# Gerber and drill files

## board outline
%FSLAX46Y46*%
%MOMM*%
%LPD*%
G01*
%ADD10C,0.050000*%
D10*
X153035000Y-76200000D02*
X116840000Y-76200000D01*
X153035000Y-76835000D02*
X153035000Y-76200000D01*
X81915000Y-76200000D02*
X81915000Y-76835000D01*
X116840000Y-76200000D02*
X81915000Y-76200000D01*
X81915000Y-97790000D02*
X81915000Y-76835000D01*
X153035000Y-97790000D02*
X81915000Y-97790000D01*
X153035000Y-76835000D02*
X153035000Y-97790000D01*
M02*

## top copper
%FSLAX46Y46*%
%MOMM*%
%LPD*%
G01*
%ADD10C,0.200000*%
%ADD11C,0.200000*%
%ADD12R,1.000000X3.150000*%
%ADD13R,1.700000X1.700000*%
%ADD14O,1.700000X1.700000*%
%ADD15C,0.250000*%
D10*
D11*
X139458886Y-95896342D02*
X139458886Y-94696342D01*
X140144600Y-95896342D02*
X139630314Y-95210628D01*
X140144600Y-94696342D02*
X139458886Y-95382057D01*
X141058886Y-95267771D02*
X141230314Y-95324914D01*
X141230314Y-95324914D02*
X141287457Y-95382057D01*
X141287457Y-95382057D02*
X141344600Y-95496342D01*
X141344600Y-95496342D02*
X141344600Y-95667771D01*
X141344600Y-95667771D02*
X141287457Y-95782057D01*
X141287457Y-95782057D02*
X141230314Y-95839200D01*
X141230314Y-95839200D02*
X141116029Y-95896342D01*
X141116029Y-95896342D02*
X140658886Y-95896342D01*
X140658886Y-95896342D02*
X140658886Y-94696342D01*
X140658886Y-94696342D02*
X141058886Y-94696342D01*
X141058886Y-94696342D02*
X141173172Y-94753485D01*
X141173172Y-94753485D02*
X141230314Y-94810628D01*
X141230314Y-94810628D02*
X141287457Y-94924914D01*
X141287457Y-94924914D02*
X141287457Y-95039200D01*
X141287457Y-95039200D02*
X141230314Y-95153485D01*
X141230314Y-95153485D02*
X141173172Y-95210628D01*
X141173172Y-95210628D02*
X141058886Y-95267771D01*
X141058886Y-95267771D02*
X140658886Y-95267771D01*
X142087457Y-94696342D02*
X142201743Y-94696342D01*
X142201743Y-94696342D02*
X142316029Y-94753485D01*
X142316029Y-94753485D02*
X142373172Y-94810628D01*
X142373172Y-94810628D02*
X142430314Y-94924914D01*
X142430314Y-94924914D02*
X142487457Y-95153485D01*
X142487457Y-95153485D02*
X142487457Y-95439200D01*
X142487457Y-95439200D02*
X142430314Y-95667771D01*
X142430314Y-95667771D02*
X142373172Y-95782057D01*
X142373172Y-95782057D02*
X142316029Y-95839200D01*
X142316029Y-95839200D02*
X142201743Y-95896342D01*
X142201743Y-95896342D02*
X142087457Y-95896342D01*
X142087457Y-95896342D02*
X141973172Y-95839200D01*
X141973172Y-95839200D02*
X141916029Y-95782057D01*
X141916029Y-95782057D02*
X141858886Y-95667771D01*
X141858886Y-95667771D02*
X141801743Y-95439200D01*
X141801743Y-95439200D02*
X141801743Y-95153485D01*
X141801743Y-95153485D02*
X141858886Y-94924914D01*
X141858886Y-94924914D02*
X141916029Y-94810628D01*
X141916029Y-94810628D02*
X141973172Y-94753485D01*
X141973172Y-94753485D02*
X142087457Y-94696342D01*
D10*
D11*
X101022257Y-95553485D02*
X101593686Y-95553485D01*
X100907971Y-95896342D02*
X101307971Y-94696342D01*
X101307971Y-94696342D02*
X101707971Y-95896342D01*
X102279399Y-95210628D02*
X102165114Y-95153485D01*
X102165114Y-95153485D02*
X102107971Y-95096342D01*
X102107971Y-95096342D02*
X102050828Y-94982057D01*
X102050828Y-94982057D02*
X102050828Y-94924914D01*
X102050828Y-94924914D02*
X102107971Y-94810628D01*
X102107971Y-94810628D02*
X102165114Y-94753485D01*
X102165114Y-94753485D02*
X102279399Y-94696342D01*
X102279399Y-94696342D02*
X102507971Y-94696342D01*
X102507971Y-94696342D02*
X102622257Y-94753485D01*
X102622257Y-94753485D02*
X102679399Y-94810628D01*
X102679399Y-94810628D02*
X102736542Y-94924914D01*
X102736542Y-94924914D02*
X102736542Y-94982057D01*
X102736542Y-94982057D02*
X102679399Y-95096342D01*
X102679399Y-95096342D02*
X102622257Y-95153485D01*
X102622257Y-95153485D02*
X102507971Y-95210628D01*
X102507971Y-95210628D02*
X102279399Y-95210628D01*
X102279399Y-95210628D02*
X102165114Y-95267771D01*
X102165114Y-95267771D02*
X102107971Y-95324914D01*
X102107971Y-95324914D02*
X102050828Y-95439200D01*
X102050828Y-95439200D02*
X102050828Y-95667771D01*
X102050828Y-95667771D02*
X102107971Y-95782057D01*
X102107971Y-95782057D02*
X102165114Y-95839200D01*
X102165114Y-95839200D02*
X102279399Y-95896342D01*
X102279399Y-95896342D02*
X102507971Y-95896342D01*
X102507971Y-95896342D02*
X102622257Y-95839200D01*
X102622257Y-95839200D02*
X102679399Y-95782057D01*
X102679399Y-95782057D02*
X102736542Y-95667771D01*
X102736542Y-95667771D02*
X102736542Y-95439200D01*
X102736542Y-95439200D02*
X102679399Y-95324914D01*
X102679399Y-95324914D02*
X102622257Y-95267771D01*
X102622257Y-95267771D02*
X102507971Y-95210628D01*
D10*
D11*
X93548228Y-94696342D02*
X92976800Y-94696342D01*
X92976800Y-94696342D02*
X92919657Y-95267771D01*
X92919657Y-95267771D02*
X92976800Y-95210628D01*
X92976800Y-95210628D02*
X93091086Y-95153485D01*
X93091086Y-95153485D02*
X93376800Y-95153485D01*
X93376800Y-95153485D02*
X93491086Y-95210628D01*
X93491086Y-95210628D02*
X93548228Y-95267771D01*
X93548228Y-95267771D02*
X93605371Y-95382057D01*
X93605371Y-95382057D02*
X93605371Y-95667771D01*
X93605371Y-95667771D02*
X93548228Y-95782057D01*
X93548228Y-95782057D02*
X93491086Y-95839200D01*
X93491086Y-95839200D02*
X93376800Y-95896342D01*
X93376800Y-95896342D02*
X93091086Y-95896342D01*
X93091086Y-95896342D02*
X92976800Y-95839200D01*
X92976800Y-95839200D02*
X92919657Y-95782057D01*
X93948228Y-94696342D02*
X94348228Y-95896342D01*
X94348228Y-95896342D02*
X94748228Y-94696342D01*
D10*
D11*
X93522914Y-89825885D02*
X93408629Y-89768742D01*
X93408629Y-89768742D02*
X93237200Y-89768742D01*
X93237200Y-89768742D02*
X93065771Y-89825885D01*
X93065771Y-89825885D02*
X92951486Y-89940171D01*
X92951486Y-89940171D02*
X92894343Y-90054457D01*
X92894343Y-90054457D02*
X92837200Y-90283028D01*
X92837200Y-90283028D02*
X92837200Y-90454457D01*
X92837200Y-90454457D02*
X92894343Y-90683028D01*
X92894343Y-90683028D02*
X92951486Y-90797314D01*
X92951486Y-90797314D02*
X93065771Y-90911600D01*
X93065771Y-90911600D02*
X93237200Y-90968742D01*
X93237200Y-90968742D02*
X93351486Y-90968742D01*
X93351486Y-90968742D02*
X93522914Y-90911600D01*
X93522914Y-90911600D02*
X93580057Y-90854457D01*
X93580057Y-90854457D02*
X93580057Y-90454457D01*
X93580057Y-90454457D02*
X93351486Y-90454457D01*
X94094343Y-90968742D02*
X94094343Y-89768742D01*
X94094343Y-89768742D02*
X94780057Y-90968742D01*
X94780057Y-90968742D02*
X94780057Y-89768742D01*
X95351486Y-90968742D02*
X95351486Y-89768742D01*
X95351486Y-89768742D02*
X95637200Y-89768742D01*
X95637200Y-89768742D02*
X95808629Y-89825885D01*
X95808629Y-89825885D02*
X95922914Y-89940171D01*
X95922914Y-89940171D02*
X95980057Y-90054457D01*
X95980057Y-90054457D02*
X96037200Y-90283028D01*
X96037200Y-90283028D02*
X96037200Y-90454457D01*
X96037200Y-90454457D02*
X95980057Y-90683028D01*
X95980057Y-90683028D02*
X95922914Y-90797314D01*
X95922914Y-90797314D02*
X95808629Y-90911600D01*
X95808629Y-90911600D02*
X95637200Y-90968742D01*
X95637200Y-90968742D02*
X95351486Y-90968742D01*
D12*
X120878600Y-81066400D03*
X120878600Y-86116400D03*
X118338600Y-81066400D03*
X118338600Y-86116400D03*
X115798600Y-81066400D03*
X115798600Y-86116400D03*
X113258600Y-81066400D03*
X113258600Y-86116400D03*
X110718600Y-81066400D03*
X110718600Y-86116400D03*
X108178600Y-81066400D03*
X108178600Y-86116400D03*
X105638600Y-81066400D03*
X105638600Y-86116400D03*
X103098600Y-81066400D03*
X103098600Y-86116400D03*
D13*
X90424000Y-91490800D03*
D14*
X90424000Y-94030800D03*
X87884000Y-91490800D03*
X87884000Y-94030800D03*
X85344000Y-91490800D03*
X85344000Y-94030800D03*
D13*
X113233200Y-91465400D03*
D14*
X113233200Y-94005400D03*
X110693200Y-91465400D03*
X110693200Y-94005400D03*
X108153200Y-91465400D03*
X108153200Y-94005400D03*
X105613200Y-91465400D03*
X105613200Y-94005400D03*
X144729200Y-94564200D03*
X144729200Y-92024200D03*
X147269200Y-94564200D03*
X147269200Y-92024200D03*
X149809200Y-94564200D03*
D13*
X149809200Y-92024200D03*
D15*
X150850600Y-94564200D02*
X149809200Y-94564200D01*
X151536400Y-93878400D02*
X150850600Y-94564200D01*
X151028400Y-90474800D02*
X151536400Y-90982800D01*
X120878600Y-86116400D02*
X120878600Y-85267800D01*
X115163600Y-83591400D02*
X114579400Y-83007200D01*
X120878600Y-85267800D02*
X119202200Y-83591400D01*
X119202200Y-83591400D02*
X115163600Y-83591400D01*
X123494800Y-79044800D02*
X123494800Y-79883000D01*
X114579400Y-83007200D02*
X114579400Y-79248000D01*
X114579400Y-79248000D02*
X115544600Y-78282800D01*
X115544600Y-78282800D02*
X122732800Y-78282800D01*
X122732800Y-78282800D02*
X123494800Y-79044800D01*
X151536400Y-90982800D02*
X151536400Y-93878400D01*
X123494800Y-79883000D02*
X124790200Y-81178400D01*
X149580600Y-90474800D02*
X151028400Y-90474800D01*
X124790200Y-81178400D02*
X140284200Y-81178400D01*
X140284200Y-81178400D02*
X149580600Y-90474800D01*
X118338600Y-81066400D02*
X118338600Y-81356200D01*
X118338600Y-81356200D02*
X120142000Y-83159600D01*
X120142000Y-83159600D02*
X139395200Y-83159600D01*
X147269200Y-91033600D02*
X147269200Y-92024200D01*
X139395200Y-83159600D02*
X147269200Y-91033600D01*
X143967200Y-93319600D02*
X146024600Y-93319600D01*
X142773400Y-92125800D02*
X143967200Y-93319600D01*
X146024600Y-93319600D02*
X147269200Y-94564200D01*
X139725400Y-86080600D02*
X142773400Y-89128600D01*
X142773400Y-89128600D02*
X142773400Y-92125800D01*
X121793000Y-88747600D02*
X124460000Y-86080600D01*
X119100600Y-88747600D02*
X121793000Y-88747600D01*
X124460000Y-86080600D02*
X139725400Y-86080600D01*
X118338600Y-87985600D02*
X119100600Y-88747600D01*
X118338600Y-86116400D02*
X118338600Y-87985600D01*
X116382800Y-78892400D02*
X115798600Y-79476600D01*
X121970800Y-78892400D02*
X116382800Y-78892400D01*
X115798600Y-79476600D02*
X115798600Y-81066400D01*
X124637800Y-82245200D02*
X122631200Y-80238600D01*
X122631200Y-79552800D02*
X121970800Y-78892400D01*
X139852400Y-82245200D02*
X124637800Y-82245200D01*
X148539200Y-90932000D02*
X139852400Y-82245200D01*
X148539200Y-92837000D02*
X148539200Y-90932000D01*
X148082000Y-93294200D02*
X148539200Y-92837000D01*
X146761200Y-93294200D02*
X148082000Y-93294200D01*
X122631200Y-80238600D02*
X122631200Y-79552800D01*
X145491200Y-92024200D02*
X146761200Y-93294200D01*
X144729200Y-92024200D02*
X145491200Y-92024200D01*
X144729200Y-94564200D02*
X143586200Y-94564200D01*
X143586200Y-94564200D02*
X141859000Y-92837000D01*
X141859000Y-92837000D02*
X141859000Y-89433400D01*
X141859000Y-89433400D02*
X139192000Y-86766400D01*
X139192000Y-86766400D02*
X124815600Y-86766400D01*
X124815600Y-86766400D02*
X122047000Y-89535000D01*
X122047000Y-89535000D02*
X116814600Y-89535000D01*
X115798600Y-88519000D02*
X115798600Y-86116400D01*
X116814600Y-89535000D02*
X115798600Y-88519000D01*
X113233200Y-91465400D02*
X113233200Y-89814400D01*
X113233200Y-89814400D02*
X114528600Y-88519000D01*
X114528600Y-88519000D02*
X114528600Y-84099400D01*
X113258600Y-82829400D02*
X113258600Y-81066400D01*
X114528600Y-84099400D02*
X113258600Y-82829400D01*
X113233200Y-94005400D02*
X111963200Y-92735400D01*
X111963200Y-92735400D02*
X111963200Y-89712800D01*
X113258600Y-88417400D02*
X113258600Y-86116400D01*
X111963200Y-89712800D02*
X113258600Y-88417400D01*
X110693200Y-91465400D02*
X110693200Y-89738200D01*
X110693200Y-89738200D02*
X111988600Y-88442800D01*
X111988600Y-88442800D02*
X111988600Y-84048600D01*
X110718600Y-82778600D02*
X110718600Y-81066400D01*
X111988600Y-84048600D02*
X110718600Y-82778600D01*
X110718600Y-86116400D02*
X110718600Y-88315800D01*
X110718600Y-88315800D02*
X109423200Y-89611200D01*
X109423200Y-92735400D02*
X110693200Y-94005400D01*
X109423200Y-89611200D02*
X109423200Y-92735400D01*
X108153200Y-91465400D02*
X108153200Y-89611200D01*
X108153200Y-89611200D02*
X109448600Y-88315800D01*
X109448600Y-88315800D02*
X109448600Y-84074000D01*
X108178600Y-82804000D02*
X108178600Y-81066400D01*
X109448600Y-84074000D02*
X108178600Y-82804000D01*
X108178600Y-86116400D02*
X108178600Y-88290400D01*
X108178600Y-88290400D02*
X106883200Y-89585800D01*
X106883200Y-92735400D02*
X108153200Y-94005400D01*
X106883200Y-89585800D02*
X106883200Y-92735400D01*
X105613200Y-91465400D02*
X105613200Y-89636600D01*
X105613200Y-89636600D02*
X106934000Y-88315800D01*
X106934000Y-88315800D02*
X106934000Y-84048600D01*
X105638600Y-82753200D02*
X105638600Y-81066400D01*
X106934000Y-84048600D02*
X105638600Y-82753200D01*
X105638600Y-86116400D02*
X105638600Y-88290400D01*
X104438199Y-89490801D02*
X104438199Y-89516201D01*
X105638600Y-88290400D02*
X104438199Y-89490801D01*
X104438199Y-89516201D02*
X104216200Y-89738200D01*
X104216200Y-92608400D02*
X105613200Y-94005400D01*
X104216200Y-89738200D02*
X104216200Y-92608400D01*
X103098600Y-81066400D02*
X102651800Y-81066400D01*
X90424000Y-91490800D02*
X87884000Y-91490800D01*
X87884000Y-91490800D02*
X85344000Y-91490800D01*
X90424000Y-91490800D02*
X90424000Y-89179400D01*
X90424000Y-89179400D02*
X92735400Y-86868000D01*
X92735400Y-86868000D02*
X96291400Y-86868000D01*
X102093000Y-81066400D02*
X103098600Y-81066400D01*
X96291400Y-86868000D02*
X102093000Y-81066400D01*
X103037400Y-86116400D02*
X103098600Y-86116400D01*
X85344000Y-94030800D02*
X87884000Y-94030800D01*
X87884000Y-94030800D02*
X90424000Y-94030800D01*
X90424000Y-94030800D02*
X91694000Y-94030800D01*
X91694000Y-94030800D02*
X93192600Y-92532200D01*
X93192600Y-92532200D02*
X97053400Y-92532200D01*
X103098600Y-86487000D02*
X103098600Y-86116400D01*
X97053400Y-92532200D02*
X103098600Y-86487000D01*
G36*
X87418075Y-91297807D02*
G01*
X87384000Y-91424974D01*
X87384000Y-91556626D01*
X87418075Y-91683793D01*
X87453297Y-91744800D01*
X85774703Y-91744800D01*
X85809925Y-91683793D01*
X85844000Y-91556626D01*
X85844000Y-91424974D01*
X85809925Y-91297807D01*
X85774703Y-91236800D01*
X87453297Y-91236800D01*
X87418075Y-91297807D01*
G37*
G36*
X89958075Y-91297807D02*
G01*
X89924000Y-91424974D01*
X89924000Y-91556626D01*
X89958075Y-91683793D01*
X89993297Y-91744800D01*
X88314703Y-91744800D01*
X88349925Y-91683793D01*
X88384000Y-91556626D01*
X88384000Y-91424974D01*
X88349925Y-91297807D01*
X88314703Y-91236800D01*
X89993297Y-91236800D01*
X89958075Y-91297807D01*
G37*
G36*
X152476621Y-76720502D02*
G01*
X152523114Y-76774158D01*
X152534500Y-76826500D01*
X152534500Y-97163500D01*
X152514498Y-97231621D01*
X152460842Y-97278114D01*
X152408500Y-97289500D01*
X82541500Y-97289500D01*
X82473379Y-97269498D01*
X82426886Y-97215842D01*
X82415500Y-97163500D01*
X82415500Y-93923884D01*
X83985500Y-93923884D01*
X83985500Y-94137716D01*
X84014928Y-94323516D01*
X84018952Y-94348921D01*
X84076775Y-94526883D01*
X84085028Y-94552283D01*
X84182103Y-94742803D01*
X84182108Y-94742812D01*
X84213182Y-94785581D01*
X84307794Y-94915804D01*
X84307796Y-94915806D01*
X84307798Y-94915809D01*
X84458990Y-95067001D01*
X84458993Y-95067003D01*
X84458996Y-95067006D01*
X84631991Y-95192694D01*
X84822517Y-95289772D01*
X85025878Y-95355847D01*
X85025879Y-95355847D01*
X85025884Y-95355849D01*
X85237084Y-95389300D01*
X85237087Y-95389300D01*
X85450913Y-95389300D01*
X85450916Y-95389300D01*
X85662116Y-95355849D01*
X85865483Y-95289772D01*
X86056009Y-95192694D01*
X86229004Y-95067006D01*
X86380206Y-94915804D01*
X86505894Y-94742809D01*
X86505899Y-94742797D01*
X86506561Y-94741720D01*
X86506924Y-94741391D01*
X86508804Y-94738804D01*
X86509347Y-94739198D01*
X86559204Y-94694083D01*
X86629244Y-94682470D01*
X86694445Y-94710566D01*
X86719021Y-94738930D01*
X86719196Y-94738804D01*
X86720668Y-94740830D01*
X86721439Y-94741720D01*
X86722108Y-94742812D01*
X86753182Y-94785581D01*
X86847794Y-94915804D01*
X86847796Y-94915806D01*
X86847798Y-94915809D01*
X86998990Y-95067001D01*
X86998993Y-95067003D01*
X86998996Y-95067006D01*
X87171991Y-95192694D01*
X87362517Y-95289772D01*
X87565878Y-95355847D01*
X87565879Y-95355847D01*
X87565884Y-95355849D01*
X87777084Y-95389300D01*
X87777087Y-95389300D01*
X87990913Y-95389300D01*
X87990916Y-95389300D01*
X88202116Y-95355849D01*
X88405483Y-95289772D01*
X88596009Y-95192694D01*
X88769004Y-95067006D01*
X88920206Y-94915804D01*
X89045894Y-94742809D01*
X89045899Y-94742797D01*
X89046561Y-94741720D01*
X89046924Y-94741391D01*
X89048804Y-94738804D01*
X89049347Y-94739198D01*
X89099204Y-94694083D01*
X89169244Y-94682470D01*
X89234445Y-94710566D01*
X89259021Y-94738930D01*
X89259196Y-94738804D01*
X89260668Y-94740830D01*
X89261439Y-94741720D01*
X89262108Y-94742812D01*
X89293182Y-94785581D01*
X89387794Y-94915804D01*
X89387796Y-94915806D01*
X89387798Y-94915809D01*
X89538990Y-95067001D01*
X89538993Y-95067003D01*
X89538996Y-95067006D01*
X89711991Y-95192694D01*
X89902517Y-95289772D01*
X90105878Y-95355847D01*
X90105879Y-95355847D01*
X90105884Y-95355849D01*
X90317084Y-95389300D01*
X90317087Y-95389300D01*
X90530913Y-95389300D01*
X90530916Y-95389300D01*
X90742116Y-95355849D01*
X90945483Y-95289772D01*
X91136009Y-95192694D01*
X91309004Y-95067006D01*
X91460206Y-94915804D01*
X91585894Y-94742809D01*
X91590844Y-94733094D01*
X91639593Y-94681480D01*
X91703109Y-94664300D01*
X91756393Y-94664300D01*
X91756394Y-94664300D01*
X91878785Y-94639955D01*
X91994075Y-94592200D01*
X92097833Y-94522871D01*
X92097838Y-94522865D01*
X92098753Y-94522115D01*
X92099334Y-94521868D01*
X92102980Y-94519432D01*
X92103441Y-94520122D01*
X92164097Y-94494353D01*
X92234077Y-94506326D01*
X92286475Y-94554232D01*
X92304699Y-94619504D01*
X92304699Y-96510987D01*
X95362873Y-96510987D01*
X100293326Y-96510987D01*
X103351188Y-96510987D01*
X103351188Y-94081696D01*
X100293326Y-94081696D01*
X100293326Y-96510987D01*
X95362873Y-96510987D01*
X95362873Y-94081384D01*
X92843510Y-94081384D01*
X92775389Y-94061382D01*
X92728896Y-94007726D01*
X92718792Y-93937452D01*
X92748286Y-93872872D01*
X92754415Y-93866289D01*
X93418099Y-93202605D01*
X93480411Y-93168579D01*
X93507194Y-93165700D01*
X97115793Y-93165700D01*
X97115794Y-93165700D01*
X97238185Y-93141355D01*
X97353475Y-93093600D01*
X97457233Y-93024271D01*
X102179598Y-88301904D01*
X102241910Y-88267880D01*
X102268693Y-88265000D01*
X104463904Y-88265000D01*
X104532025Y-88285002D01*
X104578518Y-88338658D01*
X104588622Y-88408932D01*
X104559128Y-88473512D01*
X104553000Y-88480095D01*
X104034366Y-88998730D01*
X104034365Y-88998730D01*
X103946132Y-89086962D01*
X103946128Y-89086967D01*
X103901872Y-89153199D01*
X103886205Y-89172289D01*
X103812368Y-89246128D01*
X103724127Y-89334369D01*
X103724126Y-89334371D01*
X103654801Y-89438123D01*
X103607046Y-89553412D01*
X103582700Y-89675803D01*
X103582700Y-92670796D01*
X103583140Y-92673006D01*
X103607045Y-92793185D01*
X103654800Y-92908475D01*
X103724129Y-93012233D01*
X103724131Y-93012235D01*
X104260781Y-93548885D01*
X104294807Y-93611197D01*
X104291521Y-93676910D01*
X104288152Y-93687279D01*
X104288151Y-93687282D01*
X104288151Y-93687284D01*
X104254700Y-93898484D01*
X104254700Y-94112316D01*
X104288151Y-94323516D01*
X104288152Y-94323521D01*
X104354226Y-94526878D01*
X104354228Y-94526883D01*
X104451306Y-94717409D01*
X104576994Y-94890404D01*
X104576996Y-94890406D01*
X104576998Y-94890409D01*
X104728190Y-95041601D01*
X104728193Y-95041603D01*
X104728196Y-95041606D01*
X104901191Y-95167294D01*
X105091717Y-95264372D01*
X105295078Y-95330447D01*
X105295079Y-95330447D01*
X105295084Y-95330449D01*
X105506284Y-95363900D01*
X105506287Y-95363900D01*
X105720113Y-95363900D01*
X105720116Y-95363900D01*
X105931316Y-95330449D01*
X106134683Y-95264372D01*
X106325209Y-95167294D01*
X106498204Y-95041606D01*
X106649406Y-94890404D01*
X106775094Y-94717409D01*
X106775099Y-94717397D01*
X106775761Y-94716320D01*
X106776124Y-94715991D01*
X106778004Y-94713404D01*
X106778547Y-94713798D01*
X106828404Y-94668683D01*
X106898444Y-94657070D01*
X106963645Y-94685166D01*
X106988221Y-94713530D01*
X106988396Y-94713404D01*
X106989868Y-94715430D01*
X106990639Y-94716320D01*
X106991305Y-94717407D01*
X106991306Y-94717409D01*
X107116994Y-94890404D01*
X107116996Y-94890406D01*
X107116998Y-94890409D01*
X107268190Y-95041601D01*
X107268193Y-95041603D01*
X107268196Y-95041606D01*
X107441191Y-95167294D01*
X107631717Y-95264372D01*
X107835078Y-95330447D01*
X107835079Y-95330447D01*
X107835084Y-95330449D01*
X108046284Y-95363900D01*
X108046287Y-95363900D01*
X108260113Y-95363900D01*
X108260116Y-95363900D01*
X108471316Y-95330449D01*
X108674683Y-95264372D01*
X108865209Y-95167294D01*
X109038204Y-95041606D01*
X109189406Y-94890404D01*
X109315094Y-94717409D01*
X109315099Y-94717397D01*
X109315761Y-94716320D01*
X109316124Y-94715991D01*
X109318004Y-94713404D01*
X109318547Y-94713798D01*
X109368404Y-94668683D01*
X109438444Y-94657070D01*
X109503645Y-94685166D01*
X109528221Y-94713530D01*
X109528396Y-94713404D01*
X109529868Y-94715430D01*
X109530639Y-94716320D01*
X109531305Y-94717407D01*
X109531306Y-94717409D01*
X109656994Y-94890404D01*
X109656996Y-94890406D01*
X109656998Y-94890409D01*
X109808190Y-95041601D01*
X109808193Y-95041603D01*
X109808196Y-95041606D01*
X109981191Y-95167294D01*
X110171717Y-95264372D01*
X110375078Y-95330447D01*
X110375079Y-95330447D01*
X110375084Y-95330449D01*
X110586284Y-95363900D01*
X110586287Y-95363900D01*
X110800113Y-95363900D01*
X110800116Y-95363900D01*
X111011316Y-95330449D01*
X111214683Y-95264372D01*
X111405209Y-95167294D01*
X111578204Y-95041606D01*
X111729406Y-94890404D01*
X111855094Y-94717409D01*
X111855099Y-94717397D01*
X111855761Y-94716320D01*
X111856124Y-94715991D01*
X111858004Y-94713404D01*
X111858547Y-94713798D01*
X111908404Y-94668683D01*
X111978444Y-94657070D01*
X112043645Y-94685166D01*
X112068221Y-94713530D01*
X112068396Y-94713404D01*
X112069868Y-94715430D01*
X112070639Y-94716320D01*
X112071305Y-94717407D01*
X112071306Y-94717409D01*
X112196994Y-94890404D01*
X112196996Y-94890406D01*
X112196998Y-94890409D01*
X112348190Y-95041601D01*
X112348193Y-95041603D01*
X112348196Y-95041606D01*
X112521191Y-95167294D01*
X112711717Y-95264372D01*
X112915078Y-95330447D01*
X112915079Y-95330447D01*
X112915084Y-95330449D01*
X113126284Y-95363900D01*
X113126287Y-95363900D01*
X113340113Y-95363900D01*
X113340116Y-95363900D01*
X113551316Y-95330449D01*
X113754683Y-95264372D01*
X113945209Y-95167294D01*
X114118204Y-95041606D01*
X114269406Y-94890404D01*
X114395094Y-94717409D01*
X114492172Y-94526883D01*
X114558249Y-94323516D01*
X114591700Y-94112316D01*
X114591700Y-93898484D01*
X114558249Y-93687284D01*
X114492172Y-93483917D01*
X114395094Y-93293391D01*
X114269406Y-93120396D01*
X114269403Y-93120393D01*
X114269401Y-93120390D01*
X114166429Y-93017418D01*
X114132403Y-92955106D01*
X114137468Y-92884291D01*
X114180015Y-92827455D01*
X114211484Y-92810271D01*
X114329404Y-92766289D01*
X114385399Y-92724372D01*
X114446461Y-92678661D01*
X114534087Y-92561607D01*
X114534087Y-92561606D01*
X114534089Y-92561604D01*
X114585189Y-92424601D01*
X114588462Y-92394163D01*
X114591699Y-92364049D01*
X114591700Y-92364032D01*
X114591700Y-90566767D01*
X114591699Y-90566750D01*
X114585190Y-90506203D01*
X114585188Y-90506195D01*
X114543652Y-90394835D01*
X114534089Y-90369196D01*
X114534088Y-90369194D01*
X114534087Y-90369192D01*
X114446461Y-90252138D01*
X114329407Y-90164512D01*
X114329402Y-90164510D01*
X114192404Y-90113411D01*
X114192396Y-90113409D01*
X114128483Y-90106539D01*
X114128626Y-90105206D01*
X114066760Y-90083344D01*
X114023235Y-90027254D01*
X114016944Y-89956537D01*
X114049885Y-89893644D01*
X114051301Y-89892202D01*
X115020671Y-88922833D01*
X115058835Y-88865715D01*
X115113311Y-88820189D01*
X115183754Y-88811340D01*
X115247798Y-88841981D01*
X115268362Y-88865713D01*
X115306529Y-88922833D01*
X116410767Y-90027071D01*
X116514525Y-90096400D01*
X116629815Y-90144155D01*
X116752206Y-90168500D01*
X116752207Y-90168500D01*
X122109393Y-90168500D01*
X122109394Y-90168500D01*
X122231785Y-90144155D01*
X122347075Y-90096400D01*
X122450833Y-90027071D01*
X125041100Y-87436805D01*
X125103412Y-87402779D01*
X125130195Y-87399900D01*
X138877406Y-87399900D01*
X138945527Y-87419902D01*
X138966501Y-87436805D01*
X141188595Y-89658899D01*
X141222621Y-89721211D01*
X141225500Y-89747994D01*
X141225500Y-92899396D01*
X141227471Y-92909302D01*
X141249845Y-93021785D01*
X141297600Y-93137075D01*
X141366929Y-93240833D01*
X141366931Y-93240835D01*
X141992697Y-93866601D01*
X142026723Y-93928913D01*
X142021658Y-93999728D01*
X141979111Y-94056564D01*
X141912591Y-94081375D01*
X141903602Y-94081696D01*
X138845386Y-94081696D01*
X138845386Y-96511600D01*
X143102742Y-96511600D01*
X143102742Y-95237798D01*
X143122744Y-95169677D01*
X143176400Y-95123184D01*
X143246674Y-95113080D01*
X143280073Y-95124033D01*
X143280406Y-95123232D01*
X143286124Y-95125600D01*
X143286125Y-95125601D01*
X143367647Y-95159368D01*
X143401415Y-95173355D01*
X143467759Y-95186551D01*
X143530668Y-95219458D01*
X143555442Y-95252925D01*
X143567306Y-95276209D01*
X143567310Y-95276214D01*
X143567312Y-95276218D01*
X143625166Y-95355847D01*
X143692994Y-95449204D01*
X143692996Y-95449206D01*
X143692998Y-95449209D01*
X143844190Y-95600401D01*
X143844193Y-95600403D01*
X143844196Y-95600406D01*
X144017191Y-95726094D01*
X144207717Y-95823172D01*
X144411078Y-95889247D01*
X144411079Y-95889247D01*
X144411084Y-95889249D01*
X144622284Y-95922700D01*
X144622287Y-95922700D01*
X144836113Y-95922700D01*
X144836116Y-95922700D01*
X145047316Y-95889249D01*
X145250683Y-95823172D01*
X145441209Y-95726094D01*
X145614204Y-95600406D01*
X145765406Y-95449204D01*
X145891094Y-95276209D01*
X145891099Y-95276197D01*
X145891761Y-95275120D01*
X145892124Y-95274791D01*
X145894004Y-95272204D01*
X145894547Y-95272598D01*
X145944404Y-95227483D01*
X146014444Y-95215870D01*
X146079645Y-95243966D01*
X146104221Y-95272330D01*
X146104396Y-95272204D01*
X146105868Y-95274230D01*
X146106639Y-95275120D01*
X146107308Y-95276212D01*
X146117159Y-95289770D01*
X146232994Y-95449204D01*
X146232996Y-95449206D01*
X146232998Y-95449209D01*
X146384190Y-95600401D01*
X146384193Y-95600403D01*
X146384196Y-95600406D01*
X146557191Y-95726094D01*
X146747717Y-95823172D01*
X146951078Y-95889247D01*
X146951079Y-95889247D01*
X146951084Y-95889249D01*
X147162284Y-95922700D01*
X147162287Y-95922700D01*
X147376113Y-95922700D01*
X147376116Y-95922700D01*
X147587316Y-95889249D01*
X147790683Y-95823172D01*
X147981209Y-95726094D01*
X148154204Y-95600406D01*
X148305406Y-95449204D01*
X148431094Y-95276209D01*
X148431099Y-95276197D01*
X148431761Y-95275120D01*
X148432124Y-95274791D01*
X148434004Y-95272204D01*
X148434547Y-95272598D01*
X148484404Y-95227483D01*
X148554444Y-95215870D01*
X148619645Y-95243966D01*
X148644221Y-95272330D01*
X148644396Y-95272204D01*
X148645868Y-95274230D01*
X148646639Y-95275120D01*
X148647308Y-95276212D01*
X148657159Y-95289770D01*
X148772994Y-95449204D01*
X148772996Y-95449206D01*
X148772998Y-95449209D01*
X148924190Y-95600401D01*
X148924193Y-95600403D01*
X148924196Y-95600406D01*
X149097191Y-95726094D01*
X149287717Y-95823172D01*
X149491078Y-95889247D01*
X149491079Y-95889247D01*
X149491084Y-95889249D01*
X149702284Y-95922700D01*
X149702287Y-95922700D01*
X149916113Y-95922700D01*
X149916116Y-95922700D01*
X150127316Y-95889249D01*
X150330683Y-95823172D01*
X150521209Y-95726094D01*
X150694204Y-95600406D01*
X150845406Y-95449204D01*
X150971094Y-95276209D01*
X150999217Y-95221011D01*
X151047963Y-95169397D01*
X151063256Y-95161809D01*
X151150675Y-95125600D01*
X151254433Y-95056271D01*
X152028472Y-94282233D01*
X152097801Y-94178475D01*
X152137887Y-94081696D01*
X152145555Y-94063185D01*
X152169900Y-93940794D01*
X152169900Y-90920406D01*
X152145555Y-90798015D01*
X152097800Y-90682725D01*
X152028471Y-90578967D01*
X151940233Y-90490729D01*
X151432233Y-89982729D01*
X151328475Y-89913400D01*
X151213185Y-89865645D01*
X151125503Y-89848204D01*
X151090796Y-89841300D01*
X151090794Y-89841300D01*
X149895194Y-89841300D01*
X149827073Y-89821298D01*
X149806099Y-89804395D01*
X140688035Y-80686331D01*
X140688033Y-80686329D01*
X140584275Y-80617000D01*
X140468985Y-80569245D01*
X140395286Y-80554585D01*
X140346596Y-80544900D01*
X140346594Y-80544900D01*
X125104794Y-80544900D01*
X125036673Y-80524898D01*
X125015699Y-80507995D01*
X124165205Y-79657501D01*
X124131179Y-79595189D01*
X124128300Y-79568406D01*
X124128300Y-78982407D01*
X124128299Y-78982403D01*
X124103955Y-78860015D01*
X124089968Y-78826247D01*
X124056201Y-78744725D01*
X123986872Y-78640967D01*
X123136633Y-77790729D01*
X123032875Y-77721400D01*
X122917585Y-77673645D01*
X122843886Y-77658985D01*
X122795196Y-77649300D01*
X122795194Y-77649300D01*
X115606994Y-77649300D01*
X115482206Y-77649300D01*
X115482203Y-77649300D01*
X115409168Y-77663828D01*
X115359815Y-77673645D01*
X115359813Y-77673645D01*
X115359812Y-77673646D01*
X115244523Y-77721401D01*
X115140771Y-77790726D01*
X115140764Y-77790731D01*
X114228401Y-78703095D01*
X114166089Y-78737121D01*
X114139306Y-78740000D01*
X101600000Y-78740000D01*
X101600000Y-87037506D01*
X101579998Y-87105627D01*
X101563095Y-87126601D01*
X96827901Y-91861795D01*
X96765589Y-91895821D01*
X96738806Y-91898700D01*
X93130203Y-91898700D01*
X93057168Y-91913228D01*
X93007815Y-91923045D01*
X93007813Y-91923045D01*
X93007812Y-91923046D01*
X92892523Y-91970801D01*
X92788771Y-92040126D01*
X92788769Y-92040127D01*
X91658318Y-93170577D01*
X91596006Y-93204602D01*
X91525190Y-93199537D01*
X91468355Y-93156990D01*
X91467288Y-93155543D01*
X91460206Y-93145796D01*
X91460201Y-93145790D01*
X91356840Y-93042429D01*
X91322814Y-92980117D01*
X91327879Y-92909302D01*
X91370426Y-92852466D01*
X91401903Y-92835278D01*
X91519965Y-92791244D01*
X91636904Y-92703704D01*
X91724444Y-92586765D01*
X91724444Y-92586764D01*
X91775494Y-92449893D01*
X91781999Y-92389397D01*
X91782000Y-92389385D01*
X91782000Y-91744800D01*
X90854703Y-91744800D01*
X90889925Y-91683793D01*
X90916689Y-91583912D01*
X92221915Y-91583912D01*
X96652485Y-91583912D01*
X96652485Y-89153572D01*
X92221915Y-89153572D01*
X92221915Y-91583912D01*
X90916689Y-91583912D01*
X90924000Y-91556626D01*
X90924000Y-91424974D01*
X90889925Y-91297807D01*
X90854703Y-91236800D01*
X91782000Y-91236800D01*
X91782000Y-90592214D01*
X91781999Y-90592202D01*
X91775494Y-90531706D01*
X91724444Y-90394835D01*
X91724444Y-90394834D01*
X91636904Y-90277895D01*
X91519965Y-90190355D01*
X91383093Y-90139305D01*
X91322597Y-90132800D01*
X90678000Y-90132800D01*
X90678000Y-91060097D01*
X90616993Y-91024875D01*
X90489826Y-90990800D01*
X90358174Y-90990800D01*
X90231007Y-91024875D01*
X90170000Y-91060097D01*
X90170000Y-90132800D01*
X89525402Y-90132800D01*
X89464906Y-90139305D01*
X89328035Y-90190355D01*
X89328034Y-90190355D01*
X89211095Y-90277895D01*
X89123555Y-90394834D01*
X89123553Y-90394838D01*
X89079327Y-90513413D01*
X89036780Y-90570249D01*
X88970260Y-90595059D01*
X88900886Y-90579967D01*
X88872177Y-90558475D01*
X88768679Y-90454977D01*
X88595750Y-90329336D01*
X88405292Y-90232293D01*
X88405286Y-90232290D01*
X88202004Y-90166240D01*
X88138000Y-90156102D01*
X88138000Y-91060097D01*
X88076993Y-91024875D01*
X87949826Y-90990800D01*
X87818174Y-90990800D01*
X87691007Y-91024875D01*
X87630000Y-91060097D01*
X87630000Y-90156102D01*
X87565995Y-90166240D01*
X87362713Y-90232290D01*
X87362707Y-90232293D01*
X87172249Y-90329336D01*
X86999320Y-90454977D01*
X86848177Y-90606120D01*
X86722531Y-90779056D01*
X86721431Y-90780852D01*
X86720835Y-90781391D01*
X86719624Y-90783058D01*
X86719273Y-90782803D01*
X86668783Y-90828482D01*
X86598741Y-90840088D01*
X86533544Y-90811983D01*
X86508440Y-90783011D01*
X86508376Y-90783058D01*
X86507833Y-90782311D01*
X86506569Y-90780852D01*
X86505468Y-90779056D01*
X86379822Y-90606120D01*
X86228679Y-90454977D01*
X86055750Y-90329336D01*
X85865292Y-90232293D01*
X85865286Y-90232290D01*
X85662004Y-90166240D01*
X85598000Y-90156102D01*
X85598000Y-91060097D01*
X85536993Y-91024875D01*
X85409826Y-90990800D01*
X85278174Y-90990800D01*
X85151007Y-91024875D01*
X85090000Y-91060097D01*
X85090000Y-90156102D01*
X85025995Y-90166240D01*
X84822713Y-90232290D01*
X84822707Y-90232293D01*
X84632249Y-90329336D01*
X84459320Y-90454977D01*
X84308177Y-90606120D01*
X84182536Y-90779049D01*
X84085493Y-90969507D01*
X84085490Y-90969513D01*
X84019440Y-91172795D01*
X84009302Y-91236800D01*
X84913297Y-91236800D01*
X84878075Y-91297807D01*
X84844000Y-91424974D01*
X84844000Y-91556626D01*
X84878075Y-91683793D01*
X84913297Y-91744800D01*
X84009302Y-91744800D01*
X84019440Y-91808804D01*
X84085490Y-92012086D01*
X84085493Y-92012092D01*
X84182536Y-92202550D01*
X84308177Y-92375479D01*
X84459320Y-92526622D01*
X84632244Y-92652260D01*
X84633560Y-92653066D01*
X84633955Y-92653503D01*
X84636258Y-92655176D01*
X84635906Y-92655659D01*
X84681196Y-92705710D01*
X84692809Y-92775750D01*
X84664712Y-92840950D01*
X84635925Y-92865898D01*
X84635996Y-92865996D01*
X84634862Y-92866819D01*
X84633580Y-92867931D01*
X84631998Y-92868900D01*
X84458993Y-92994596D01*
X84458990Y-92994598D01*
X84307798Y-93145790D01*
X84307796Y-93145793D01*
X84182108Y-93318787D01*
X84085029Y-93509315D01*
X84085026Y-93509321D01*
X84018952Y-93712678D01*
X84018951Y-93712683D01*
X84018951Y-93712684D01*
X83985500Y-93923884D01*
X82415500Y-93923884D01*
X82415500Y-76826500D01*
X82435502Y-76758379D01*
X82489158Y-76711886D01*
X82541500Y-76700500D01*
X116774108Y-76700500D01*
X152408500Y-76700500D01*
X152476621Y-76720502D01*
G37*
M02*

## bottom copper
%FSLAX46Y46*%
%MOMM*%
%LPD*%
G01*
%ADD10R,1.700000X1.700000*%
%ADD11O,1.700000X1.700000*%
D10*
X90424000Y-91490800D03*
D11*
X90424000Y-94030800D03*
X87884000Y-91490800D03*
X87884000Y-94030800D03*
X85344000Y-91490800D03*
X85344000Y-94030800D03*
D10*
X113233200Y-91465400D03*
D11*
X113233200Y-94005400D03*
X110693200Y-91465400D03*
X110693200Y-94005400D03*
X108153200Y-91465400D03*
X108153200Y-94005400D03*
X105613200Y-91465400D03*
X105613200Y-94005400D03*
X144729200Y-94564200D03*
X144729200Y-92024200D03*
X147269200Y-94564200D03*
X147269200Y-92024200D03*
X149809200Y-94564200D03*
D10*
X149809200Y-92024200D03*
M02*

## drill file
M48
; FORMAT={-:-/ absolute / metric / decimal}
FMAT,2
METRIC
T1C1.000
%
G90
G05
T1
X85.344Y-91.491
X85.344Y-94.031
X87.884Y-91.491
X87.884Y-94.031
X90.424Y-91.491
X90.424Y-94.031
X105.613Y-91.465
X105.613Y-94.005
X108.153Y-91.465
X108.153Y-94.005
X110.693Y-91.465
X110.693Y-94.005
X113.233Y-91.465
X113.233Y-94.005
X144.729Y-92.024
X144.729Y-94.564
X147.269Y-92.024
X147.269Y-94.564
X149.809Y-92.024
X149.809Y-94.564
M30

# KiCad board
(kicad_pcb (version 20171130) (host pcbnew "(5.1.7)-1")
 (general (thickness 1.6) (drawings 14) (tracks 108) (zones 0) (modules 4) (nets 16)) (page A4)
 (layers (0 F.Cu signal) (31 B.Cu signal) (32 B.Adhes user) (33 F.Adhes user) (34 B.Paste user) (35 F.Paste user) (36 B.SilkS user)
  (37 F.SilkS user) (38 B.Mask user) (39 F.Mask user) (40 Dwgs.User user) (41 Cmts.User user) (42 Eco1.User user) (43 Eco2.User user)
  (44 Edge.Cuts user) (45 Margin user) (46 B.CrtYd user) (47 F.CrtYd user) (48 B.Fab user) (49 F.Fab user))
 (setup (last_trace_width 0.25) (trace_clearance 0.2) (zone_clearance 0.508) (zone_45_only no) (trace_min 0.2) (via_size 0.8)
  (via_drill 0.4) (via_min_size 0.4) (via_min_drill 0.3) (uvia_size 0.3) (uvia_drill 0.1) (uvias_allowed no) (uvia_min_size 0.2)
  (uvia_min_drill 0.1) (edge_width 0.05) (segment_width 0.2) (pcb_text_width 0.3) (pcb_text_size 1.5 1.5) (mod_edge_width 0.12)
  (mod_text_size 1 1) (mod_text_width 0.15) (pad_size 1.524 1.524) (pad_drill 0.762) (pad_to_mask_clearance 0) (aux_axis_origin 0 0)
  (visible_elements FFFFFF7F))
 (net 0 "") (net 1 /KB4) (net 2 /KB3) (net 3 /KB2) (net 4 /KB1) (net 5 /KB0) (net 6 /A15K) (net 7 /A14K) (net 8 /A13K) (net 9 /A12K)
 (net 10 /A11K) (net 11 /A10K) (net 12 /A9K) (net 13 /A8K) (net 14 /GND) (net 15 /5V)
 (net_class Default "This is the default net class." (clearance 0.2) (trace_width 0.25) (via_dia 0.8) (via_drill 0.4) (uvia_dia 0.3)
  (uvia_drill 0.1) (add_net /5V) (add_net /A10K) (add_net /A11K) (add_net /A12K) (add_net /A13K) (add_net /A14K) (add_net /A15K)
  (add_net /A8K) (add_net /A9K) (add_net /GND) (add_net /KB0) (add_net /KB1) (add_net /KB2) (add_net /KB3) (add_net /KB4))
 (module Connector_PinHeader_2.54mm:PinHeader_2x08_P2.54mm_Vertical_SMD (layer F.Cu) (at 111.9886 83.5914 270)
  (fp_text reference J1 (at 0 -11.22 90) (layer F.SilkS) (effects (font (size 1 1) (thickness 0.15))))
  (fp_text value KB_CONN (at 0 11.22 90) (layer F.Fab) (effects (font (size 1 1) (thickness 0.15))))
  (pad 1 smd rect (at -2.525 -8.89 270) (size 3.15 1) (layers F.Cu F.Paste F.Mask))
  (pad 2 smd rect (at 2.525 -8.89 270) (size 3.15 1) (layers F.Cu F.Paste F.Mask) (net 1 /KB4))
  (pad 3 smd rect (at -2.525 -6.35 270) (size 3.15 1) (layers F.Cu F.Paste F.Mask) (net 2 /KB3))
  (pad 4 smd rect (at 2.525 -6.35 270) (size 3.15 1) (layers F.Cu F.Paste F.Mask) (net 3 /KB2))
  (pad 5 smd rect (at -2.525 -3.81 270) (size 3.15 1) (layers F.Cu F.Paste F.Mask) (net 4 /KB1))
  (pad 6 smd rect (at 2.525 -3.81 270) (size 3.15 1) (layers F.Cu F.Paste F.Mask) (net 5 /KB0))
  (pad 7 smd rect (at -2.525 -1.27 270) (size 3.15 1) (layers F.Cu F.Paste F.Mask) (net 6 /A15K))
  (pad 8 smd rect (at 2.525 -1.27 270) (size 3.15 1) (layers F.Cu F.Paste F.Mask) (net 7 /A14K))
  (pad 9 smd rect (at -2.525 1.27 270) (size 3.15 1) (layers F.Cu F.Paste F.Mask) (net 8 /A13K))
  (pad 10 smd rect (at 2.525 1.27 270) (size 3.15 1) (layers F.Cu F.Paste F.Mask) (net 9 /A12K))
  (pad 11 smd rect (at -2.525 3.81 270) (size 3.15 1) (layers F.Cu F.Paste F.Mask) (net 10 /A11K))
  (pad 12 smd rect (at 2.525 3.81 270) (size 3.15 1) (layers F.Cu F.Paste F.Mask) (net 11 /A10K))
  (pad 13 smd rect (at -2.525 6.35 270) (size 3.15 1) (layers F.Cu F.Paste F.Mask) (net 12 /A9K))
  (pad 14 smd rect (at 2.525 6.35 270) (size 3.15 1) (layers F.Cu F.Paste F.Mask) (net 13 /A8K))
  (pad 15 smd rect (at -2.525 8.89 270) (size 3.15 1) (layers F.Cu F.Paste F.Mask) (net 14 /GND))
  (pad 16 smd rect (at 2.525 8.89 270) (size 3.15 1) (layers F.Cu F.Paste F.Mask) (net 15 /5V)))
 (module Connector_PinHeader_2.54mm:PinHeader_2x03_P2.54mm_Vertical (layer F.Cu) (at 90.424 91.4908 270)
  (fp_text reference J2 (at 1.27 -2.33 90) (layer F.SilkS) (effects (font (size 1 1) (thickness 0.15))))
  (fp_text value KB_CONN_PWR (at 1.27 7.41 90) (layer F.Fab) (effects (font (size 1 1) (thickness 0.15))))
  (pad 1 thru_hole rect (at 0 0 270) (size 1.7 1.7) (drill 1) (layers *.Cu *.Mask) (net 14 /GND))
  (pad 2 thru_hole oval (at 2.54 0 270) (size 1.7 1.7) (drill 1) (layers *.Cu *.Mask) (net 15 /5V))
  (pad 3 thru_hole oval (at 0 2.54 270) (size 1.7 1.7) (drill 1) (layers *.Cu *.Mask) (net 14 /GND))
  (pad 4 thru_hole oval (at 2.54 2.54 270) (size 1.7 1.7) (drill 1) (layers *.Cu *.Mask) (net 15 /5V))
  (pad 5 thru_hole oval (at 0 5.08 270) (size 1.7 1.7) (drill 1) (layers *.Cu *.Mask) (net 14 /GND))
  (pad 6 thru_hole oval (at 2.54 5.08 270) (size 1.7 1.7) (drill 1) (layers *.Cu *.Mask) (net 15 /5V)))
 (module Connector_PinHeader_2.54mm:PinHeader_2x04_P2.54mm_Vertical (layer F.Cu) (at 113.2332 91.4654 270)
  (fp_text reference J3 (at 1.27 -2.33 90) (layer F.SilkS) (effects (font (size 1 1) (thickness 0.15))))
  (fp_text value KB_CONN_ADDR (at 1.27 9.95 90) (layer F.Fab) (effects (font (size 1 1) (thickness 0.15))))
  (pad 1 thru_hole rect (at 0 0 270) (size 1.7 1.7) (drill 1) (layers *.Cu *.Mask) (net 6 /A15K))
  (pad 2 thru_hole oval (at 2.54 0 270) (size 1.7 1.7) (drill 1) (layers *.Cu *.Mask) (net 7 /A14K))
  (pad 3 thru_hole oval (at 0 2.54 270) (size 1.7 1.7) (drill 1) (layers *.Cu *.Mask) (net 8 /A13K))
  (pad 4 thru_hole oval (at 2.54 2.54 270) (size 1.7 1.7) (drill 1) (layers *.Cu *.Mask) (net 9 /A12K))
  (pad 5 thru_hole oval (at 0 5.08 270) (size 1.7 1.7) (drill 1) (layers *.Cu *.Mask) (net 10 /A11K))
  (pad 6 thru_hole oval (at 2.54 5.08 270) (size 1.7 1.7) (drill 1) (layers *.Cu *.Mask) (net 11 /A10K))
  (pad 7 thru_hole oval (at 0 7.62 270) (size 1.7 1.7) (drill 1) (layers *.Cu *.Mask) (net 12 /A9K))
  (pad 8 thru_hole oval (at 2.54 7.62 270) (size 1.7 1.7) (drill 1) (layers *.Cu *.Mask) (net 13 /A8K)))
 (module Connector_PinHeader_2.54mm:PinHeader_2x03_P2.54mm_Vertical (layer F.Cu) (at 149.8092 92.0242 270)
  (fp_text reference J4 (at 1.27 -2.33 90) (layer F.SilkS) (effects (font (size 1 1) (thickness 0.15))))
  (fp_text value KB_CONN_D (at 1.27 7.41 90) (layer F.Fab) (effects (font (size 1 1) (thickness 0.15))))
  (pad 6 thru_hole oval (at 2.54 5.08 270) (size 1.7 1.7) (drill 1) (layers *.Cu *.Mask) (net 5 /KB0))
  (pad 5 thru_hole oval (at 0 5.08 270) (size 1.7 1.7) (drill 1) (layers *.Cu *.Mask) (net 4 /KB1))
  (pad 4 thru_hole oval (at 2.54 2.54 270) (size 1.7 1.7) (drill 1) (layers *.Cu *.Mask) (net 3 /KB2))
  (pad 3 thru_hole oval (at 0 2.54 270) (size 1.7 1.7) (drill 1) (layers *.Cu *.Mask) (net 2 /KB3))
  (pad 2 thru_hole oval (at 2.54 0 270) (size 1.7 1.7) (drill 1) (layers *.Cu *.Mask) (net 1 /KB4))
  (pad 1 thru_hole rect (at 0 0 270) (size 1.7 1.7) (drill 1) (layers *.Cu *.Mask)))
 (gr_line (start 153.035 76.2) (end 116.84 76.2) (layer Edge.Cuts) (width 0.05))
 (gr_line (start 153.035 76.835) (end 153.035 76.2) (layer Edge.Cuts) (width 0.05))
 (gr_line (start 81.915 76.2) (end 81.915 76.835) (layer Edge.Cuts) (width 0.05))
 (gr_line (start 116.84 76.2) (end 81.915 76.2) (layer Edge.Cuts) (width 0.05))
 (gr_line (start 81.915 97.79) (end 81.915 76.835) (layer Edge.Cuts) (width 0.05))
 (gr_line (start 153.035 97.79) (end 81.915 97.79) (layer Edge.Cuts) (width 0.05))
 (gr_line (start 153.035 76.835) (end 153.035 97.79) (layer Edge.Cuts) (width 0.05))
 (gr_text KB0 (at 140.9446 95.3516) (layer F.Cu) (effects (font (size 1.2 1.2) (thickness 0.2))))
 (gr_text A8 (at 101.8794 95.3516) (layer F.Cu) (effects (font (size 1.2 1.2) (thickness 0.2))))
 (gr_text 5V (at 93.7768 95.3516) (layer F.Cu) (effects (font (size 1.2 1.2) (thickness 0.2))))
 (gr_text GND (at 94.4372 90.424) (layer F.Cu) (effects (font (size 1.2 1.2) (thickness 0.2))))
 (segment (start 150.8506 94.5642) (end 149.8092 94.5642) (width 0.25) (layer F.Cu) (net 1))
 (segment (start 151.5364 93.8784) (end 150.8506 94.5642) (width 0.25) (layer F.Cu) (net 1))
 (segment (start 151.0284 90.4748) (end 151.5364 90.9828) (width 0.25) (layer F.Cu) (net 1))
 (segment (start 120.8786 86.1164) (end 120.8786 85.2678) (width 0.25) (layer F.Cu) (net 1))
 (segment (start 115.1636 83.5914) (end 114.5794 83.0072) (width 0.25) (layer F.Cu) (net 1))
 (segment (start 120.8786 85.2678) (end 119.2022 83.5914) (width 0.25) (layer F.Cu) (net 1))
 (segment (start 119.2022 83.5914) (end 115.1636 83.5914) (width 0.25) (layer F.Cu) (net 1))
 (segment (start 123.4948 79.0448) (end 123.4948 79.883) (width 0.25) (layer F.Cu) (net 1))
 (segment (start 114.5794 83.0072) (end 114.5794 79.248) (width 0.25) (layer F.Cu) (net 1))
 (segment (start 114.5794 79.248) (end 115.5446 78.2828) (width 0.25) (layer F.Cu) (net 1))
 (segment (start 115.5446 78.2828) (end 122.7328 78.2828) (width 0.25) (layer F.Cu) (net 1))
 (segment (start 122.7328 78.2828) (end 123.4948 79.0448) (width 0.25) (layer F.Cu) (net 1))
 (segment (start 151.5364 90.9828) (end 151.5364 93.8784) (width 0.25) (layer F.Cu) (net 1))
 (segment (start 123.4948 79.883) (end 124.7902 81.1784) (width 0.25) (layer F.Cu) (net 1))
 (segment (start 149.5806 90.4748) (end 151.0284 90.4748) (width 0.25) (layer F.Cu) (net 1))
 (segment (start 124.7902 81.1784) (end 140.2842 81.1784) (width 0.25) (layer F.Cu) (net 1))
 (segment (start 140.2842 81.1784) (end 149.5806 90.4748) (width 0.25) (layer F.Cu) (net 1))
 (segment (start 118.3386 81.0664) (end 118.3386 81.3562) (width 0.25) (layer F.Cu) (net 2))
 (segment (start 118.3386 81.3562) (end 120.142 83.1596) (width 0.25) (layer F.Cu) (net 2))
 (segment (start 120.142 83.1596) (end 139.3952 83.1596) (width 0.25) (layer F.Cu) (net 2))
 (segment (start 147.2692 91.0336) (end 147.2692 92.0242) (width 0.25) (layer F.Cu) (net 2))
 (segment (start 139.3952 83.1596) (end 147.2692 91.0336) (width 0.25) (layer F.Cu) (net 2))
 (segment (start 143.9672 93.3196) (end 146.0246 93.3196) (width 0.25) (layer F.Cu) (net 3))
 (segment (start 142.7734 92.1258) (end 143.9672 93.3196) (width 0.25) (layer F.Cu) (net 3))
 (segment (start 146.0246 93.3196) (end 147.2692 94.5642) (width 0.25) (layer F.Cu) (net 3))
 (segment (start 139.7254 86.0806) (end 142.7734 89.1286) (width 0.25) (layer F.Cu) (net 3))
 (segment (start 142.7734 89.1286) (end 142.7734 92.1258) (width 0.25) (layer F.Cu) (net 3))
 (segment (start 121.793 88.7476) (end 124.46 86.0806) (width 0.25) (layer F.Cu) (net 3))
 (segment (start 119.1006 88.7476) (end 121.793 88.7476) (width 0.25) (layer F.Cu) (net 3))
 (segment (start 124.46 86.0806) (end 139.7254 86.0806) (width 0.25) (layer F.Cu) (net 3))
 (segment (start 118.3386 87.9856) (end 119.1006 88.7476) (width 0.25) (layer F.Cu) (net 3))
 (segment (start 118.3386 86.1164) (end 118.3386 87.9856) (width 0.25) (layer F.Cu) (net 3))
 (segment (start 116.3828 78.8924) (end 115.7986 79.4766) (width 0.25) (layer F.Cu) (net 4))
 (segment (start 121.9708 78.8924) (end 116.3828 78.8924) (width 0.25) (layer F.Cu) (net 4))
 (segment (start 115.7986 79.4766) (end 115.7986 81.0664) (width 0.25) (layer F.Cu) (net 4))
 (segment (start 124.6378 82.2452) (end 122.6312 80.2386) (width 0.25) (layer F.Cu) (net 4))
 (segment (start 122.6312 79.5528) (end 121.9708 78.8924) (width 0.25) (layer F.Cu) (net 4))
 (segment (start 139.8524 82.2452) (end 124.6378 82.2452) (width 0.25) (layer F.Cu) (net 4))
 (segment (start 148.5392 90.932) (end 139.8524 82.2452) (width 0.25) (layer F.Cu) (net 4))
 (segment (start 148.5392 92.837) (end 148.5392 90.932) (width 0.25) (layer F.Cu) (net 4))
 (segment (start 148.082 93.2942) (end 148.5392 92.837) (width 0.25) (layer F.Cu) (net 4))
 (segment (start 146.7612 93.2942) (end 148.082 93.2942) (width 0.25) (layer F.Cu) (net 4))
 (segment (start 122.6312 80.2386) (end 122.6312 79.5528) (width 0.25) (layer F.Cu) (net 4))
 (segment (start 145.4912 92.0242) (end 146.7612 93.2942) (width 0.25) (layer F.Cu) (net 4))
 (segment (start 144.7292 92.0242) (end 145.4912 92.0242) (width 0.25) (layer F.Cu) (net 4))
 (segment (start 144.7292 94.5642) (end 143.5862 94.5642) (width 0.25) (layer F.Cu) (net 5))
 (segment (start 143.5862 94.5642) (end 141.859 92.837) (width 0.25) (layer F.Cu) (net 5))
 (segment (start 141.859 92.837) (end 141.859 89.4334) (width 0.25) (layer F.Cu) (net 5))
 (segment (start 141.859 89.4334) (end 139.192 86.7664) (width 0.25) (layer F.Cu) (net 5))
 (segment (start 139.192 86.7664) (end 124.8156 86.7664) (width 0.25) (layer F.Cu) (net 5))
 (segment (start 124.8156 86.7664) (end 122.047 89.535) (width 0.25) (layer F.Cu) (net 5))
 (segment (start 122.047 89.535) (end 116.8146 89.535) (width 0.25) (layer F.Cu) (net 5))
 (segment (start 115.7986 88.519) (end 115.7986 86.1164) (width 0.25) (layer F.Cu) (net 5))
 (segment (start 116.8146 89.535) (end 115.7986 88.519) (width 0.25) (layer F.Cu) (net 5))
 (segment (start 113.2332 91.4654) (end 113.2332 89.8144) (width 0.25) (layer F.Cu) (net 6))
 (segment (start 113.2332 89.8144) (end 114.5286 88.519) (width 0.25) (layer F.Cu) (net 6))
 (segment (start 114.5286 88.519) (end 114.5286 84.0994) (width 0.25) (layer F.Cu) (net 6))
 (segment (start 113.2586 82.8294) (end 113.2586 81.0664) (width 0.25) (layer F.Cu) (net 6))
 (segment (start 114.5286 84.0994) (end 113.2586 82.8294) (width 0.25) (layer F.Cu) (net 6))
 (segment (start 113.2332 94.0054) (end 111.9632 92.7354) (width 0.25) (layer F.Cu) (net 7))
 (segment (start 111.9632 92.7354) (end 111.9632 89.7128) (width 0.25) (layer F.Cu) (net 7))
 (segment (start 113.2586 88.4174) (end 113.2586 86.1164) (width 0.25) (layer F.Cu) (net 7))
 (segment (start 111.9632 89.7128) (end 113.2586 88.4174) (width 0.25) (layer F.Cu) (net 7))
 (segment (start 110.6932 91.4654) (end 110.6932 89.7382) (width 0.25) (layer F.Cu) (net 8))
 (segment (start 110.6932 89.7382) (end 111.9886 88.4428) (width 0.25) (layer F.Cu) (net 8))
 (segment (start 111.9886 88.4428) (end 111.9886 84.0486) (width 0.25) (layer F.Cu) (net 8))
 (segment (start 110.7186 82.7786) (end 110.7186 81.0664) (width 0.25) (layer F.Cu) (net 8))
 (segment (start 111.9886 84.0486) (end 110.7186 82.7786) (width 0.25) (layer F.Cu) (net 8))
 (segment (start 110.7186 86.1164) (end 110.7186 88.3158) (width 0.25) (layer F.Cu) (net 9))
 (segment (start 110.7186 88.3158) (end 109.4232 89.6112) (width 0.25) (layer F.Cu) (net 9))
 (segment (start 109.4232 92.7354) (end 110.6932 94.0054) (width 0.25) (layer F.Cu) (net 9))
 (segment (start 109.4232 89.6112) (end 109.4232 92.7354) (width 0.25) (layer F.Cu) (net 9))
 (segment (start 108.1532 91.4654) (end 108.1532 89.6112) (width 0.25) (layer F.Cu) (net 10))
 (segment (start 108.1532 89.6112) (end 109.4486 88.3158) (width 0.25) (layer F.Cu) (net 10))
 (segment (start 109.4486 88.3158) (end 109.4486 84.074) (width 0.25) (layer F.Cu) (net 10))
 (segment (start 108.1786 82.804) (end 108.1786 81.0664) (width 0.25) (layer F.Cu) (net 10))
 (segment (start 109.4486 84.074) (end 108.1786 82.804) (width 0.25) (layer F.Cu) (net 10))
 (segment (start 108.1786 86.1164) (end 108.1786 88.2904) (width 0.25) (layer F.Cu) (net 11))
 (segment (start 108.1786 88.2904) (end 106.8832 89.5858) (width 0.25) (layer F.Cu) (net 11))
 (segment (start 106.8832 92.7354) (end 108.1532 94.0054) (width 0.25) (layer F.Cu) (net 11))
 (segment (start 106.8832 89.5858) (end 106.8832 92.7354) (width 0.25) (layer F.Cu) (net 11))
 (segment (start 105.6132 91.4654) (end 105.6132 89.6366) (width 0.25) (layer F.Cu) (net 12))
 (segment (start 105.6132 89.6366) (end 106.934 88.3158) (width 0.25) (layer F.Cu) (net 12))
 (segment (start 106.934 88.3158) (end 106.934 84.0486) (width 0.25) (layer F.Cu) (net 12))
 (segment (start 105.6386 82.7532) (end 105.6386 81.0664) (width 0.25) (layer F.Cu) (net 12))
 (segment (start 106.934 84.0486) (end 105.6386 82.7532) (width 0.25) (layer F.Cu) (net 12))
 (segment (start 105.6386 86.1164) (end 105.6386 88.2904) (width 0.25) (layer F.Cu) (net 13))
 (segment (start 104.438199 89.490801) (end 104.438199 89.516201) (width 0.25) (layer F.Cu) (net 13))
 (segment (start 105.6386 88.2904) (end 104.438199 89.490801) (width 0.25) (layer F.Cu) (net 13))
 (segment (start 104.438199 89.516201) (end 104.2162 89.7382) (width 0.25) (layer F.Cu) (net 13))
 (segment (start 104.2162 92.6084) (end 105.6132 94.0054) (width 0.25) (layer F.Cu) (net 13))
 (segment (start 104.2162 89.7382) (end 104.2162 92.6084) (width 0.25) (layer F.Cu) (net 13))
 (segment (start 103.0986 81.0664) (end 102.6518 81.0664) (width 0.25) (layer F.Cu) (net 14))
 (segment (start 90.424 91.4908) (end 87.884 91.4908) (width 0.25) (layer F.Cu) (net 14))
 (segment (start 87.884 91.4908) (end 85.344 91.4908) (width 0.25) (layer F.Cu) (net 14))
 (segment (start 90.424 91.4908) (end 90.424 89.1794) (width 0.25) (layer F.Cu) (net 14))
 (segment (start 90.424 89.1794) (end 92.7354 86.868) (width 0.25) (layer F.Cu) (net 14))
 (segment (start 92.7354 86.868) (end 96.2914 86.868) (width 0.25) (layer F.Cu) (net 14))
 (segment (start 102.093 81.0664) (end 103.0986 81.0664) (width 0.25) (layer F.Cu) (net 14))
 (segment (start 96.2914 86.868) (end 102.093 81.0664) (width 0.25) (layer F.Cu) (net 14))
 (segment (start 103.0374 86.1164) (end 103.0986 86.1164) (width 0.25) (layer F.Cu) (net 15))
 (segment (start 85.344 94.0308) (end 87.884 94.0308) (width 0.25) (layer F.Cu) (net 15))
 (segment (start 87.884 94.0308) (end 90.424 94.0308) (width 0.25) (layer F.Cu) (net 15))
 (segment (start 90.424 94.0308) (end 91.694 94.0308) (width 0.25) (layer F.Cu) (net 15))
 (segment (start 91.694 94.0308) (end 93.1926 92.5322) (width 0.25) (layer F.Cu) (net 15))
 (segment (start 93.1926 92.5322) (end 97.0534 92.5322) (width 0.25) (layer F.Cu) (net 15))
 (segment (start 103.0986 86.487) (end 103.0986 86.1164) (width 0.25) (layer F.Cu) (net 15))
 (segment (start 97.0534 92.5322) (end 103.0986 86.487) (width 0.25) (layer F.Cu) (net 15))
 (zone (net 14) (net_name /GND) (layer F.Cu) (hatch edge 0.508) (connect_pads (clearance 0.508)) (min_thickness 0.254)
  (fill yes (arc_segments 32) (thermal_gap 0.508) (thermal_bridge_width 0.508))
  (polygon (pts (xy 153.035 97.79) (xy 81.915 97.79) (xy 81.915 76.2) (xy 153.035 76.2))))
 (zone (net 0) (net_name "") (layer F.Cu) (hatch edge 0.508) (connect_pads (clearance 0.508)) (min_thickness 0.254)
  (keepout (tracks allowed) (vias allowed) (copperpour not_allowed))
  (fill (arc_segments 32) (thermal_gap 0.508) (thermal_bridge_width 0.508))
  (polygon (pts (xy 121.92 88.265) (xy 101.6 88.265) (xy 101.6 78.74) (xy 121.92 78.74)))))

